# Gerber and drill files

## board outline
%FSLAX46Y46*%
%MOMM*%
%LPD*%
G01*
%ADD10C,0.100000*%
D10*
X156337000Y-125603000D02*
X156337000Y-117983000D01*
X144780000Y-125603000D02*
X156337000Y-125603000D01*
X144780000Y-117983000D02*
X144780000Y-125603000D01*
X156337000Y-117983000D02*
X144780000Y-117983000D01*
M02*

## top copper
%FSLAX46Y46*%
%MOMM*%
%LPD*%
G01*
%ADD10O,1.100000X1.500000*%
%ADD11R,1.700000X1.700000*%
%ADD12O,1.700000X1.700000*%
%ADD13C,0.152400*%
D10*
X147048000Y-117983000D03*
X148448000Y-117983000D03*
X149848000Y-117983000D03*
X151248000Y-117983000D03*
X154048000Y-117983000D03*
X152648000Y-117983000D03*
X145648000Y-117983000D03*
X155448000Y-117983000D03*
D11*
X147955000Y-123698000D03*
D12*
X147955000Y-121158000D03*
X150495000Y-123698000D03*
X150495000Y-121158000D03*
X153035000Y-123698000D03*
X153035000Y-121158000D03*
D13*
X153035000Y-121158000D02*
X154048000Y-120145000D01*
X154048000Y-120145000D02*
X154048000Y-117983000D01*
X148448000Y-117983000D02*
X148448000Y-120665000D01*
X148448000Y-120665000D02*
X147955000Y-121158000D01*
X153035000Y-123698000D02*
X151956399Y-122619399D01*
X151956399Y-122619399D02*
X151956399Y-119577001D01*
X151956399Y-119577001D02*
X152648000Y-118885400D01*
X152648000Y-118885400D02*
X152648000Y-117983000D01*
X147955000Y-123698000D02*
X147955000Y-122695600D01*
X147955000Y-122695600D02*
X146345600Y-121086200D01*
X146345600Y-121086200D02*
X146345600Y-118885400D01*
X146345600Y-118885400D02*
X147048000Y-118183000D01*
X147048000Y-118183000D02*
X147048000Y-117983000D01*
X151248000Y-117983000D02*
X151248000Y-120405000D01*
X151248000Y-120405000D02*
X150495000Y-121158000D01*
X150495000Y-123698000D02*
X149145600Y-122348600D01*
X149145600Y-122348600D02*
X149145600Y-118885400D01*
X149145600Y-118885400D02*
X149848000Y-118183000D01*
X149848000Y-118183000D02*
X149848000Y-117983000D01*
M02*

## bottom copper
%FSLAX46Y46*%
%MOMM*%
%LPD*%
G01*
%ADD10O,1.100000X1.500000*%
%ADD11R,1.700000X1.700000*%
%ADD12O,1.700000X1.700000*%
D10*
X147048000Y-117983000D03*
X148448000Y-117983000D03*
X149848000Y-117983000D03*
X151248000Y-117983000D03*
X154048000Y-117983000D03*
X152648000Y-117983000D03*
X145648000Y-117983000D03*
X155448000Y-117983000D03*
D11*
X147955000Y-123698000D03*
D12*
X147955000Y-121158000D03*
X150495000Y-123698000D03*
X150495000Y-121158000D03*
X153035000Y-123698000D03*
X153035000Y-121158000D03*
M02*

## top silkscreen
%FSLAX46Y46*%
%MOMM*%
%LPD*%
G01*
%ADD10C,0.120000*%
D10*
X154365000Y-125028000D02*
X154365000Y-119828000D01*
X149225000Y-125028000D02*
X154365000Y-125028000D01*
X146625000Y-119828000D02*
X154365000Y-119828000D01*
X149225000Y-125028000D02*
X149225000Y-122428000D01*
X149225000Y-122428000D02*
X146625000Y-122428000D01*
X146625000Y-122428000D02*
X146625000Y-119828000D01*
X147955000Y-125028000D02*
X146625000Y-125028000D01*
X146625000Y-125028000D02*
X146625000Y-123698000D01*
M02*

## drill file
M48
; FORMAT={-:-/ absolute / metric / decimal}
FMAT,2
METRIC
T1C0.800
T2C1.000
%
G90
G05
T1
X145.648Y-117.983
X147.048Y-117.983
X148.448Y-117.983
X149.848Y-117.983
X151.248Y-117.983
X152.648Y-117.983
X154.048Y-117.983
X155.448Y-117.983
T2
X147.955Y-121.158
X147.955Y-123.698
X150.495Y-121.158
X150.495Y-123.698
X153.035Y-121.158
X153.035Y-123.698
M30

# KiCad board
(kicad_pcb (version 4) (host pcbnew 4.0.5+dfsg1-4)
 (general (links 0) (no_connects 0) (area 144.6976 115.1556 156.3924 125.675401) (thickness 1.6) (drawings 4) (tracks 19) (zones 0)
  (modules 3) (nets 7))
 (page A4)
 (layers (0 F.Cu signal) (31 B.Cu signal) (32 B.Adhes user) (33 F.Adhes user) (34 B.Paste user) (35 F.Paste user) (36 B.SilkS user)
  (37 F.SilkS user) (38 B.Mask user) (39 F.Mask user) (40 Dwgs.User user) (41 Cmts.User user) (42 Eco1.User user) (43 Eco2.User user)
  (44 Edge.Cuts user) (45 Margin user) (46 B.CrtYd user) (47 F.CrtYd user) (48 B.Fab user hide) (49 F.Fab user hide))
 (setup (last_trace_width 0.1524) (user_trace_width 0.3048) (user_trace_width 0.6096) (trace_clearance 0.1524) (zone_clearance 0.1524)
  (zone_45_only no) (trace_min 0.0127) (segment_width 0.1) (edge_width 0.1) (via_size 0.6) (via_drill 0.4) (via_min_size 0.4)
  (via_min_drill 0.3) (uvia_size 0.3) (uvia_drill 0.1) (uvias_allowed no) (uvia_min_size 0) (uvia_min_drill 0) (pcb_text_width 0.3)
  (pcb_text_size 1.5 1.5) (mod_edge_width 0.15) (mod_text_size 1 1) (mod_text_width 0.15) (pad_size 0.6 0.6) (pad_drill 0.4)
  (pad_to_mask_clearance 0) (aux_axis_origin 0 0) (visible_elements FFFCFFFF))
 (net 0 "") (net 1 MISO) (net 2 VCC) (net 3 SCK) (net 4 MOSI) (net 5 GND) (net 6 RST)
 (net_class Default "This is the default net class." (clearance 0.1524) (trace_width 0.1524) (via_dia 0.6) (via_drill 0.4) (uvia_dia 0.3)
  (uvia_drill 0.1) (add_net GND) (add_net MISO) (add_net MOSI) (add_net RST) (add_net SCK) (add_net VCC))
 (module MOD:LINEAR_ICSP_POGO (layer F.Cu) (at 150.548 116.583)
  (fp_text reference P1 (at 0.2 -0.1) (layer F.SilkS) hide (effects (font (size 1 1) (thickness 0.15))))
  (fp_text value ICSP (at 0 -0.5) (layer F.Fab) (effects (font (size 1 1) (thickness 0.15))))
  (pad 1 thru_hole oval (at -3.5 1.4) (size 1.1 1.5) (drill 0.8) (layers *.Cu *.Mask) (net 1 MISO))
  (pad 2 thru_hole oval (at -2.1 1.4) (size 1.1 1.5) (drill 0.8) (layers *.Cu *.Mask) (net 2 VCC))
  (pad 3 thru_hole oval (at -0.7 1.4) (size 1.1 1.5) (drill 0.8) (layers *.Cu *.Mask) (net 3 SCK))
  (pad 4 thru_hole oval (at 0.7 1.4) (size 1.1 1.5) (drill 0.8) (layers *.Cu *.Mask) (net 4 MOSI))
  (pad 6 thru_hole oval (at 3.5 1.4) (size 1.1 1.5) (drill 0.8) (layers *.Cu *.Mask) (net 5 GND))
  (pad 5 thru_hole oval (at 2.1 1.4) (size 1.1 1.5) (drill 0.8) (layers *.Cu *.Mask) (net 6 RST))
  (pad NC1 thru_hole oval (at -4.9 1.4) (size 1.1 1.5) (drill 0.8) (layers *.Cu *.Mask))
  (pad NC2 thru_hole oval (at 4.9 1.4) (size 1.1 1.5) (drill 0.8) (layers *.Cu *.Mask)))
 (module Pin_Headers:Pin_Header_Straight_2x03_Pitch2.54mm (layer F.Cu) (at 147.955 123.698 90)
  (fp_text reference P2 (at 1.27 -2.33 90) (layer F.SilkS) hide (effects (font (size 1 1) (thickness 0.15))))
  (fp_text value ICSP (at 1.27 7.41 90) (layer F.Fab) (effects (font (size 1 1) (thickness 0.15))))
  (fp_line (start -1.33 6.41) (end 3.87 6.41) (layer F.SilkS) (width 0.12))
  (fp_line (start -1.33 1.27) (end -1.33 6.41) (layer F.SilkS) (width 0.12))
  (fp_line (start 3.87 -1.33) (end 3.87 6.41) (layer F.SilkS) (width 0.12))
  (fp_line (start -1.33 1.27) (end 1.27 1.27) (layer F.SilkS) (width 0.12))
  (fp_line (start 1.27 1.27) (end 1.27 -1.33) (layer F.SilkS) (width 0.12))
  (fp_line (start 1.27 -1.33) (end 3.87 -1.33) (layer F.SilkS) (width 0.12))
  (fp_line (start -1.33 0) (end -1.33 -1.33) (layer F.SilkS) (width 0.12))
  (fp_line (start -1.33 -1.33) (end 0 -1.33) (layer F.SilkS) (width 0.12))
  (pad 1 thru_hole rect (at 0 0 90) (size 1.7 1.7) (drill 1) (layers *.Cu *.Mask) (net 1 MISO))
  (pad 2 thru_hole oval (at 2.54 0 90) (size 1.7 1.7) (drill 1) (layers *.Cu *.Mask) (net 2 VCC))
  (pad 3 thru_hole oval (at 0 2.54 90) (size 1.7 1.7) (drill 1) (layers *.Cu *.Mask) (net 3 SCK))
  (pad 4 thru_hole oval (at 2.54 2.54 90) (size 1.7 1.7) (drill 1) (layers *.Cu *.Mask) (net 4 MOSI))
  (pad 5 thru_hole oval (at 0 5.08 90) (size 1.7 1.7) (drill 1) (layers *.Cu *.Mask) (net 6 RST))
  (pad 6 thru_hole oval (at 2.54 5.08 90) (size 1.7 1.7) (drill 1) (layers *.Cu *.Mask) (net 5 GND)))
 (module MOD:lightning (layer B.Cu) (at 154.94 122.682)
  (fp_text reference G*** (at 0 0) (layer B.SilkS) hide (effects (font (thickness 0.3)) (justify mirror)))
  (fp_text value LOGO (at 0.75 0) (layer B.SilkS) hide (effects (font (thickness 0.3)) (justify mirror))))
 (gr_line (start 156.337 125.603) (end 156.337 117.983) (layer Edge.Cuts) (width 0.1))
 (gr_line (start 144.78 125.603) (end 156.337 125.603) (layer Edge.Cuts) (width 0.1))
 (gr_line (start 144.78 117.983) (end 144.78 125.603) (layer Edge.Cuts) (width 0.1))
 (gr_line (start 156.337 117.983) (end 144.78 117.983) (layer Edge.Cuts) (width 0.1))
 (segment (start 153.035 121.158) (end 154.048 120.145) (width 0.1524) (layer F.Cu) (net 5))
 (segment (start 154.048 120.145) (end 154.048 117.983) (width 0.1524) (layer F.Cu) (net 5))
 (segment (start 148.448 117.983) (end 148.448 120.665) (width 0.1524) (layer F.Cu) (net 2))
 (segment (start 148.448 120.665) (end 147.955 121.158) (width 0.1524) (layer F.Cu) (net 2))
 (segment (start 153.035 123.698) (end 151.956399 122.619399) (width 0.1524) (layer F.Cu) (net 6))
 (segment (start 151.956399 122.619399) (end 151.956399 119.577001) (width 0.1524) (layer F.Cu) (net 6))
 (segment (start 151.956399 119.577001) (end 152.648 118.8854) (width 0.1524) (layer F.Cu) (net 6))
 (segment (start 152.648 118.8854) (end 152.648 117.983) (width 0.1524) (layer F.Cu) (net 6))
 (segment (start 147.955 123.698) (end 147.955 122.6956) (width 0.1524) (layer F.Cu) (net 1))
 (segment (start 147.955 122.6956) (end 146.3456 121.0862) (width 0.1524) (layer F.Cu) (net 1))
 (segment (start 146.3456 121.0862) (end 146.3456 118.8854) (width 0.1524) (layer F.Cu) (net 1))
 (segment (start 146.3456 118.8854) (end 147.048 118.183) (width 0.1524) (layer F.Cu) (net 1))
 (segment (start 147.048 118.183) (end 147.048 117.983) (width 0.1524) (layer F.Cu) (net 1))
 (segment (start 151.248 117.983) (end 151.248 120.405) (width 0.1524) (layer F.Cu) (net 4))
 (segment (start 151.248 120.405) (end 150.495 121.158) (width 0.1524) (layer F.Cu) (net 4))
 (segment (start 150.495 123.698) (end 149.1456 122.3486) (width 0.1524) (layer F.Cu) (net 3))
 (segment (start 149.1456 122.3486) (end 149.1456 118.8854) (width 0.1524) (layer F.Cu) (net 3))
 (segment (start 149.1456 118.8854) (end 149.848 118.183) (width 0.1524) (layer F.Cu) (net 3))
 (segment (start 149.848 118.183) (end 149.848 117.983) (width 0.1524) (layer F.Cu) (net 3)))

